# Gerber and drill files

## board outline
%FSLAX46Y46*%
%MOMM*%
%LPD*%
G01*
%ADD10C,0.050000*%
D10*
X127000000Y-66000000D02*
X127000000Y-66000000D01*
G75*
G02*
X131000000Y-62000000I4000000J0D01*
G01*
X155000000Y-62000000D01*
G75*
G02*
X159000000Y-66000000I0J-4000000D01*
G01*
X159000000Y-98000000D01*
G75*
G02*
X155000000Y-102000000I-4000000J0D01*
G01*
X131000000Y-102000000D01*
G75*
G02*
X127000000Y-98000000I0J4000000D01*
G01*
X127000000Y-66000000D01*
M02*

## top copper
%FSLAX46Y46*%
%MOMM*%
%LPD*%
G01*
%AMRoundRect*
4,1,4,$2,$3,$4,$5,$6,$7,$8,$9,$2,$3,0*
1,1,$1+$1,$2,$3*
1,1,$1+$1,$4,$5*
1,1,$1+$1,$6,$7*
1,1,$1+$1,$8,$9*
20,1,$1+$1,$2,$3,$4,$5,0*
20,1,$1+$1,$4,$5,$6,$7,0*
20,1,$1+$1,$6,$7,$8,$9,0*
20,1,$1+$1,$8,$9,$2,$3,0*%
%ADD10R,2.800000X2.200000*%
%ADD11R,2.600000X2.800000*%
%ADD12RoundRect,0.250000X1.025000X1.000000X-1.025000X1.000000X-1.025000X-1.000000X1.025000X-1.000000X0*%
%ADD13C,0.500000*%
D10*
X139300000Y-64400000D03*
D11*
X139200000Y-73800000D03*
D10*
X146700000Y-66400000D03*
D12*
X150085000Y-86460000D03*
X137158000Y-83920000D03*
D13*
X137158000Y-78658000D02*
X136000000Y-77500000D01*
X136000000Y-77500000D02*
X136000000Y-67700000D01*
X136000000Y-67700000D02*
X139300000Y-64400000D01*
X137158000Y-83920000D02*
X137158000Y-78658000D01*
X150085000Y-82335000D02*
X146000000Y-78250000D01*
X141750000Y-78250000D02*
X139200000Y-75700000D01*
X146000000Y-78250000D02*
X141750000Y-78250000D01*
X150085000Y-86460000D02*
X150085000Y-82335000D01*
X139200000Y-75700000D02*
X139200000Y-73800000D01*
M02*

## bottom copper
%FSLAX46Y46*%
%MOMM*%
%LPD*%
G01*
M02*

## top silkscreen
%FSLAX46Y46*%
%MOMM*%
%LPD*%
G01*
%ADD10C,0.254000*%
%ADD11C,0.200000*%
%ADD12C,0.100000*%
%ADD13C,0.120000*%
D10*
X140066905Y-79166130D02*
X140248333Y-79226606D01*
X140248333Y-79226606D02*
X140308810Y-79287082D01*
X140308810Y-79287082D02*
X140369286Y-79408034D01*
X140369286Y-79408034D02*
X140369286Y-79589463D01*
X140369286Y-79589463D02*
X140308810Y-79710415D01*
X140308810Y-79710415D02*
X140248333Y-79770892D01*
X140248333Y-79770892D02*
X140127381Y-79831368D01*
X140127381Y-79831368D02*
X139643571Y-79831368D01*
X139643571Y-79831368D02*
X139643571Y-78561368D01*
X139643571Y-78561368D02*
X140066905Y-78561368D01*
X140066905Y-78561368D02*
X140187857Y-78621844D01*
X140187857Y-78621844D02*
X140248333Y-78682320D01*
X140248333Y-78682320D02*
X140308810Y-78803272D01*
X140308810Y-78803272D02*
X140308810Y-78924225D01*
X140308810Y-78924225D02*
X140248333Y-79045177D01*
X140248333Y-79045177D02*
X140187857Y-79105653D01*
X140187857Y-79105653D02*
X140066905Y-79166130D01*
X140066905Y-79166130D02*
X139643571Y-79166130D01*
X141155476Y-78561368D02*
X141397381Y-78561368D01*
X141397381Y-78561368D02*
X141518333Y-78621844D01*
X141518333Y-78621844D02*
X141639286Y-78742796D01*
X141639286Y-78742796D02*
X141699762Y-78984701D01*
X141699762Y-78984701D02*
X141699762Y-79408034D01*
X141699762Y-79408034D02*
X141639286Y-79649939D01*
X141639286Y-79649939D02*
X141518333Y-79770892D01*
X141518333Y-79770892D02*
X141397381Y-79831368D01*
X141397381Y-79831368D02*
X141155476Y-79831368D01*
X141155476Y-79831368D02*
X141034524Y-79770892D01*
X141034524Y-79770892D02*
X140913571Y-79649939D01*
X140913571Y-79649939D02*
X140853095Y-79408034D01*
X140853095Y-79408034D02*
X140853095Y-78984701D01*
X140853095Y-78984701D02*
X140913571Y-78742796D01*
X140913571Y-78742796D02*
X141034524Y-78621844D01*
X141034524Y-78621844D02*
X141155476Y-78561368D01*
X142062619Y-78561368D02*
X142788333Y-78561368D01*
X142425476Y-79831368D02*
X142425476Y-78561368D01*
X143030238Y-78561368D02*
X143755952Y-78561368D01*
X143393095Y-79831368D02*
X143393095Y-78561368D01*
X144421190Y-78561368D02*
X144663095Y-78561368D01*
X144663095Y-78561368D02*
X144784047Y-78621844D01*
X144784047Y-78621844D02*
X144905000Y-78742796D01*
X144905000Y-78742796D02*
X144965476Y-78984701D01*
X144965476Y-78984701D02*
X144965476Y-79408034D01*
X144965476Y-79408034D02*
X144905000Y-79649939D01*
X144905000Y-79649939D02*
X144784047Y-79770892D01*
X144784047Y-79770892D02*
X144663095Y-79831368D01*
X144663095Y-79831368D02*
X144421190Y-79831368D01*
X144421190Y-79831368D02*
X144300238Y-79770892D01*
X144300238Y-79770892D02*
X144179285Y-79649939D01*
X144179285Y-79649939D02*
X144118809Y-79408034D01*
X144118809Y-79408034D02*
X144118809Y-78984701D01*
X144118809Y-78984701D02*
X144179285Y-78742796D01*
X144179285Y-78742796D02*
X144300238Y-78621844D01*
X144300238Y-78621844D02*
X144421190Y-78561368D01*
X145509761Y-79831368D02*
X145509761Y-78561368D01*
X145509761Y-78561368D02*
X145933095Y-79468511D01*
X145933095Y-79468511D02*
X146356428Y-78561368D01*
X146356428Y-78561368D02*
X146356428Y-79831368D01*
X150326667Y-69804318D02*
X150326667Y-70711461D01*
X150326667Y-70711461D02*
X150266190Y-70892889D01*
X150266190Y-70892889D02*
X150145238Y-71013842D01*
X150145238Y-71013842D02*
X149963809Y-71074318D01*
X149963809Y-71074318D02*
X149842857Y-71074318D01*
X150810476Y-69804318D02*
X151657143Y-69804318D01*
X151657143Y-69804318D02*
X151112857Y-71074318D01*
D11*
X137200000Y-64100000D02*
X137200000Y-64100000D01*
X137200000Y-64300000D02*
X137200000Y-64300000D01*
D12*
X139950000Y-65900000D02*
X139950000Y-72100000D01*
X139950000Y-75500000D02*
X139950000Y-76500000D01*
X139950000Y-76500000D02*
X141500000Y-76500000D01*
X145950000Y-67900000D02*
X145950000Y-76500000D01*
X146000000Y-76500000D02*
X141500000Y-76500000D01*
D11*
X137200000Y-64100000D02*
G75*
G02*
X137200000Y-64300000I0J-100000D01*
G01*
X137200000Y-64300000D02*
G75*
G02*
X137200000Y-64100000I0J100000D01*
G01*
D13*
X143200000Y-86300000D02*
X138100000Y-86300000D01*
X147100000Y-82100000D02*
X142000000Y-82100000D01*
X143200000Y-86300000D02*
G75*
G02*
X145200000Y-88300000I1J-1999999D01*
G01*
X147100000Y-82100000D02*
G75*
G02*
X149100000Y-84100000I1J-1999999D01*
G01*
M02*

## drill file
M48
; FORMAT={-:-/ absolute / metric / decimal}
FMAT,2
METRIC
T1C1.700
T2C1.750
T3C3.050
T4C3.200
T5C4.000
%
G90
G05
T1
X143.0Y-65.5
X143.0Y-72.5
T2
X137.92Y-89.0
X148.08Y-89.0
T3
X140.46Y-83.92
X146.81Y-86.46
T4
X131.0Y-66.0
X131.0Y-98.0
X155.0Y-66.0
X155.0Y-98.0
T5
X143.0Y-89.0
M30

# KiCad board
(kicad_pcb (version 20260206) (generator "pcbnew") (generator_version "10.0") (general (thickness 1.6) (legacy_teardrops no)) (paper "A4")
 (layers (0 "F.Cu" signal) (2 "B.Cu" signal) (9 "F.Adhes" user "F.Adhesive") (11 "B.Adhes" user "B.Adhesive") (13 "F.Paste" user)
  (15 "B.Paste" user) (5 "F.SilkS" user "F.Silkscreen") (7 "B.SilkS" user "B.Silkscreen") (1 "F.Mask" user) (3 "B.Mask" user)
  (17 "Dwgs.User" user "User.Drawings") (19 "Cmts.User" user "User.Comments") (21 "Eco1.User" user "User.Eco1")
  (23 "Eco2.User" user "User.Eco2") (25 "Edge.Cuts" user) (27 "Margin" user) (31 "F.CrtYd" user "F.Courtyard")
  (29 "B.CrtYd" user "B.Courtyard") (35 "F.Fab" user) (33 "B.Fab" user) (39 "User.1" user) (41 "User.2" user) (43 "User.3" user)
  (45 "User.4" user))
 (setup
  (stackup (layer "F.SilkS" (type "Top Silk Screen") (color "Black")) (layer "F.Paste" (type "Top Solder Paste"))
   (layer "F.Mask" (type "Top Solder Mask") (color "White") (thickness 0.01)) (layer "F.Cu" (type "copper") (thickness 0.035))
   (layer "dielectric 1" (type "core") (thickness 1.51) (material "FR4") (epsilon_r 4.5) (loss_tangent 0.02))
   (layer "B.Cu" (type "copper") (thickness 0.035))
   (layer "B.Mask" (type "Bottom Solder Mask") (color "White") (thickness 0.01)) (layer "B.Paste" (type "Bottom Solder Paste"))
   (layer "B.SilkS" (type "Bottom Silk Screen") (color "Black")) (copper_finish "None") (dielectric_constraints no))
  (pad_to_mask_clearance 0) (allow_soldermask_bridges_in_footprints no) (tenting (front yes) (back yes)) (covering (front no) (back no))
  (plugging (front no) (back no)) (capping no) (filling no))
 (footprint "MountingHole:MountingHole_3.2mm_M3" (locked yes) (layer "F.Cu") (at 155 66)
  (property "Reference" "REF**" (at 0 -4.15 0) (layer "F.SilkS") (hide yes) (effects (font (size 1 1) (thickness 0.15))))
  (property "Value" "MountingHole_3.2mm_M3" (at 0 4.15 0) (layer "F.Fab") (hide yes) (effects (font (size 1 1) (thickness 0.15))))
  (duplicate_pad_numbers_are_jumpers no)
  (pad "" np_thru_hole circle (at 0 0) (size 3.2 3.2) (drill 3.2) (layers "*.Cu" "*.Mask")))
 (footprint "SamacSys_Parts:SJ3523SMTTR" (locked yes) (layer "F.Cu") (at 143 62 -90)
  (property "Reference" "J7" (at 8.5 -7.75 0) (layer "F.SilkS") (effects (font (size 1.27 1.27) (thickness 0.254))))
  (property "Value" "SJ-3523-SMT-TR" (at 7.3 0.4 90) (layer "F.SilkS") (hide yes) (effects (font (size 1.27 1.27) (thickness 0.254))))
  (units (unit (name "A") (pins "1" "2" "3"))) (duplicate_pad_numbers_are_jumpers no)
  (fp_line (start 2.1 5.8) (end 2.1 5.8) (stroke (width 0.2) (type solid)) (layer "F.SilkS"))
  (fp_line (start 2.3 5.8) (end 2.3 5.8) (stroke (width 0.2) (type solid)) (layer "F.SilkS"))
  (fp_line (start 3.9 3.05) (end 10.1 3.05) (stroke (width 0.1) (type solid)) (layer "F.SilkS"))
  (fp_line (start 13.5 3.05) (end 14.5 3.05) (stroke (width 0.1) (type solid)) (layer "F.SilkS"))
  (fp_line (start 14.5 3.05) (end 14.5 1.5) (stroke (width 0.1) (type solid)) (layer "F.SilkS"))
  (fp_line (start 5.9 -2.95) (end 14.5 -2.95) (stroke (width 0.1) (type solid)) (layer "F.SilkS"))
  (fp_line (start 14.5 -3) (end 14.5 1.5) (stroke (width 0.1) (type solid)) (layer "F.SilkS"))
  (fp_arc (start 2.1 5.8) (mid 2.2 5.7) (end 2.3 5.8) (stroke (width 0.2) (type solid)) (layer "F.SilkS"))
  (fp_arc (start 2.3 5.8) (mid 2.2 5.9) (end 2.1 5.8) (stroke (width 0.2) (type solid)) (layer "F.SilkS"))
  (pad "" np_thru_hole circle (at 3.5 0 270) (size 1.7 1.7) (drill 1.7) (layers "*.Cu" "*.Mask"))
  (pad "" np_thru_hole circle (at 10.5 0 270) (size 1.7 1.7) (drill 1.7) (layers "*.Cu" "*.Mask"))
  (pad "1" smd rect (at 2.4 3.7 270) (size 2.2 2.8) (layers "F.Cu" "F.Mask" "F.Paste") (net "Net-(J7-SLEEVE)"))
  (pad "2" smd rect (at 11.8 3.8) (size 2.6 2.8) (layers "F.Cu" "F.Mask" "F.Paste") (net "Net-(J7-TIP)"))
  (pad "3" smd rect (at 4.4 -3.7 270) (size 2.2 2.8) (layers "F.Cu" "F.Mask" "F.Paste") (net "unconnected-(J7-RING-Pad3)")))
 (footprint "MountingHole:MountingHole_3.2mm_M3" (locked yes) (layer "F.Cu") (at 155 98)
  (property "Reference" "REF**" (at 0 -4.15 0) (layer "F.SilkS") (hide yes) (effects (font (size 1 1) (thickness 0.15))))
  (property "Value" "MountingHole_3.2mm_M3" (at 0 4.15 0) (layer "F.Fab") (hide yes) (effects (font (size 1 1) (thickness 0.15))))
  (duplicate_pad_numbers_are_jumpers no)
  (pad "" np_thru_hole circle (at 0 0) (size 3.2 3.2) (drill 3.2) (layers "*.Cu" "*.Mask")))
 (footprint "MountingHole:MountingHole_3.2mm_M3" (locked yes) (layer "F.Cu") (at 131 66)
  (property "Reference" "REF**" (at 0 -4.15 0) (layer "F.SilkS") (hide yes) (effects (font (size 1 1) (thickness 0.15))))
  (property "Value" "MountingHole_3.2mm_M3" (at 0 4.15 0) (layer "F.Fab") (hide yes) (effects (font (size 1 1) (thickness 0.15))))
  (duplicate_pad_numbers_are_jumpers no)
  (pad "" np_thru_hole circle (at 0 0) (size 3.2 3.2) (drill 3.2) (layers "*.Cu" "*.Mask")))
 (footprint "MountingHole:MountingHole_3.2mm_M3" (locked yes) (layer "F.Cu") (at 131 98)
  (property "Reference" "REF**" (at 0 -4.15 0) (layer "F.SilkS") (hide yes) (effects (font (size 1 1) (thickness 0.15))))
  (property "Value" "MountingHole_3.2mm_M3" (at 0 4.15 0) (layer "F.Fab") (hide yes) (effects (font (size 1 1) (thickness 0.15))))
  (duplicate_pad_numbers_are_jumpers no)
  (pad "" np_thru_hole circle (at 0 0) (size 3.2 3.2) (drill 3.2) (layers "*.Cu" "*.Mask")))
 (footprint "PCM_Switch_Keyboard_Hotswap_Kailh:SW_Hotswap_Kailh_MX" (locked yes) (layer "B.Cu") (at 143 89 180)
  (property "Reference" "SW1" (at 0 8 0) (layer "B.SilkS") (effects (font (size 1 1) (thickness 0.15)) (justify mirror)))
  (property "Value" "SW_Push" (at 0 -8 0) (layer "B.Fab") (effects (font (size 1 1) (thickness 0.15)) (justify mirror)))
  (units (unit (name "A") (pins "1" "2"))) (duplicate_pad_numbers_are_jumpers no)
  (fp_line (start -0.2 2.7) (end 4.9 2.7) (stroke (width 0.12) (type solid)) (layer "F.SilkS"))
  (fp_line (start -4.1 6.9) (end 1 6.9) (stroke (width 0.12) (type solid)) (layer "F.SilkS"))
  (fp_arc (start -0.2 2.7) (mid -1.614214 2.114214) (end -2.2 0.7) (stroke (width 0.12) (type solid)) (layer "F.SilkS"))
  (fp_arc (start -4.1 6.9) (mid -5.514214 6.314214) (end -6.1 4.9) (stroke (width 0.12) (type solid)) (layer "F.SilkS"))
  (pad "" np_thru_hole circle (at -5.08 0 180) (size 1.75 1.75) (drill 1.75) (layers "*.Cu" "*.Mask"))
  (pad "" np_thru_hole circle (at -3.81 2.54 180) (size 3.05 3.05) (drill 3.05) (layers "*.Cu" "*.Mask"))
  (pad "" np_thru_hole circle (at 0 0 180) (size 4 4) (drill 4) (layers "*.Cu" "*.Mask"))
  (pad "" np_thru_hole circle (at 2.54 5.08 180) (size 3.05 3.05) (drill 3.05) (layers "*.Cu" "*.Mask"))
  (pad "" np_thru_hole circle (at 5.08 0 180) (size 1.75 1.75) (drill 1.75) (layers "*.Cu" "*.Mask"))
  (pad "1" smd roundrect (at -7.085 2.54 180) (size 2.55 2.5) (layers "F.Cu" "F.Mask" "F.Paste") (roundrect_rratio 0.1) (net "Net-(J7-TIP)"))
  (pad "2" smd roundrect (at 5.842 5.08 180) (size 2.55 2.5) (layers "F.Cu" "F.Mask" "F.Paste") (roundrect_rratio 0.1)
   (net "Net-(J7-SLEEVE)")))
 (gr_rect (start 127 62) (end 159 102) (radius 4) (stroke (width 0.05) (type solid)) (fill no) (locked yes) (layer "Edge.Cuts"))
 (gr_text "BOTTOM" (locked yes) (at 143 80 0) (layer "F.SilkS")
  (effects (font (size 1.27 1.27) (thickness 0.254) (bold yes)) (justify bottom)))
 (segment (start 137.158 78.658) (end 136 77.5) (width 0.5) (locked yes) (layer "F.Cu") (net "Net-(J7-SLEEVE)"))
 (segment (start 136 77.5) (end 136 67.7) (width 0.5) (locked yes) (layer "F.Cu") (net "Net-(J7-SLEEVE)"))
 (segment (start 136 67.7) (end 139.3 64.4) (width 0.5) (locked yes) (layer "F.Cu") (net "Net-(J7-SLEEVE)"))
 (segment (start 137.158 83.92) (end 137.158 78.658) (width 0.5) (locked yes) (layer "F.Cu") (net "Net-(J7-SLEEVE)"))
 (segment (start 150.085 82.335) (end 146 78.25) (width 0.5) (locked yes) (layer "F.Cu") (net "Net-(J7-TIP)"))
 (segment (start 141.75 78.25) (end 139.2 75.7) (width 0.5) (locked yes) (layer "F.Cu") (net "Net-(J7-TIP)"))
 (segment (start 146 78.25) (end 141.75 78.25) (width 0.5) (locked yes) (layer "F.Cu") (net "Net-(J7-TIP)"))
 (segment (start 150.085 86.46) (end 150.085 82.335) (width 0.5) (locked yes) (layer "F.Cu") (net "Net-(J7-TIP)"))
 (segment (start 139.2 75.7) (end 139.2 73.8) (width 0.5) (locked yes) (layer "F.Cu") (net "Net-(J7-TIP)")))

